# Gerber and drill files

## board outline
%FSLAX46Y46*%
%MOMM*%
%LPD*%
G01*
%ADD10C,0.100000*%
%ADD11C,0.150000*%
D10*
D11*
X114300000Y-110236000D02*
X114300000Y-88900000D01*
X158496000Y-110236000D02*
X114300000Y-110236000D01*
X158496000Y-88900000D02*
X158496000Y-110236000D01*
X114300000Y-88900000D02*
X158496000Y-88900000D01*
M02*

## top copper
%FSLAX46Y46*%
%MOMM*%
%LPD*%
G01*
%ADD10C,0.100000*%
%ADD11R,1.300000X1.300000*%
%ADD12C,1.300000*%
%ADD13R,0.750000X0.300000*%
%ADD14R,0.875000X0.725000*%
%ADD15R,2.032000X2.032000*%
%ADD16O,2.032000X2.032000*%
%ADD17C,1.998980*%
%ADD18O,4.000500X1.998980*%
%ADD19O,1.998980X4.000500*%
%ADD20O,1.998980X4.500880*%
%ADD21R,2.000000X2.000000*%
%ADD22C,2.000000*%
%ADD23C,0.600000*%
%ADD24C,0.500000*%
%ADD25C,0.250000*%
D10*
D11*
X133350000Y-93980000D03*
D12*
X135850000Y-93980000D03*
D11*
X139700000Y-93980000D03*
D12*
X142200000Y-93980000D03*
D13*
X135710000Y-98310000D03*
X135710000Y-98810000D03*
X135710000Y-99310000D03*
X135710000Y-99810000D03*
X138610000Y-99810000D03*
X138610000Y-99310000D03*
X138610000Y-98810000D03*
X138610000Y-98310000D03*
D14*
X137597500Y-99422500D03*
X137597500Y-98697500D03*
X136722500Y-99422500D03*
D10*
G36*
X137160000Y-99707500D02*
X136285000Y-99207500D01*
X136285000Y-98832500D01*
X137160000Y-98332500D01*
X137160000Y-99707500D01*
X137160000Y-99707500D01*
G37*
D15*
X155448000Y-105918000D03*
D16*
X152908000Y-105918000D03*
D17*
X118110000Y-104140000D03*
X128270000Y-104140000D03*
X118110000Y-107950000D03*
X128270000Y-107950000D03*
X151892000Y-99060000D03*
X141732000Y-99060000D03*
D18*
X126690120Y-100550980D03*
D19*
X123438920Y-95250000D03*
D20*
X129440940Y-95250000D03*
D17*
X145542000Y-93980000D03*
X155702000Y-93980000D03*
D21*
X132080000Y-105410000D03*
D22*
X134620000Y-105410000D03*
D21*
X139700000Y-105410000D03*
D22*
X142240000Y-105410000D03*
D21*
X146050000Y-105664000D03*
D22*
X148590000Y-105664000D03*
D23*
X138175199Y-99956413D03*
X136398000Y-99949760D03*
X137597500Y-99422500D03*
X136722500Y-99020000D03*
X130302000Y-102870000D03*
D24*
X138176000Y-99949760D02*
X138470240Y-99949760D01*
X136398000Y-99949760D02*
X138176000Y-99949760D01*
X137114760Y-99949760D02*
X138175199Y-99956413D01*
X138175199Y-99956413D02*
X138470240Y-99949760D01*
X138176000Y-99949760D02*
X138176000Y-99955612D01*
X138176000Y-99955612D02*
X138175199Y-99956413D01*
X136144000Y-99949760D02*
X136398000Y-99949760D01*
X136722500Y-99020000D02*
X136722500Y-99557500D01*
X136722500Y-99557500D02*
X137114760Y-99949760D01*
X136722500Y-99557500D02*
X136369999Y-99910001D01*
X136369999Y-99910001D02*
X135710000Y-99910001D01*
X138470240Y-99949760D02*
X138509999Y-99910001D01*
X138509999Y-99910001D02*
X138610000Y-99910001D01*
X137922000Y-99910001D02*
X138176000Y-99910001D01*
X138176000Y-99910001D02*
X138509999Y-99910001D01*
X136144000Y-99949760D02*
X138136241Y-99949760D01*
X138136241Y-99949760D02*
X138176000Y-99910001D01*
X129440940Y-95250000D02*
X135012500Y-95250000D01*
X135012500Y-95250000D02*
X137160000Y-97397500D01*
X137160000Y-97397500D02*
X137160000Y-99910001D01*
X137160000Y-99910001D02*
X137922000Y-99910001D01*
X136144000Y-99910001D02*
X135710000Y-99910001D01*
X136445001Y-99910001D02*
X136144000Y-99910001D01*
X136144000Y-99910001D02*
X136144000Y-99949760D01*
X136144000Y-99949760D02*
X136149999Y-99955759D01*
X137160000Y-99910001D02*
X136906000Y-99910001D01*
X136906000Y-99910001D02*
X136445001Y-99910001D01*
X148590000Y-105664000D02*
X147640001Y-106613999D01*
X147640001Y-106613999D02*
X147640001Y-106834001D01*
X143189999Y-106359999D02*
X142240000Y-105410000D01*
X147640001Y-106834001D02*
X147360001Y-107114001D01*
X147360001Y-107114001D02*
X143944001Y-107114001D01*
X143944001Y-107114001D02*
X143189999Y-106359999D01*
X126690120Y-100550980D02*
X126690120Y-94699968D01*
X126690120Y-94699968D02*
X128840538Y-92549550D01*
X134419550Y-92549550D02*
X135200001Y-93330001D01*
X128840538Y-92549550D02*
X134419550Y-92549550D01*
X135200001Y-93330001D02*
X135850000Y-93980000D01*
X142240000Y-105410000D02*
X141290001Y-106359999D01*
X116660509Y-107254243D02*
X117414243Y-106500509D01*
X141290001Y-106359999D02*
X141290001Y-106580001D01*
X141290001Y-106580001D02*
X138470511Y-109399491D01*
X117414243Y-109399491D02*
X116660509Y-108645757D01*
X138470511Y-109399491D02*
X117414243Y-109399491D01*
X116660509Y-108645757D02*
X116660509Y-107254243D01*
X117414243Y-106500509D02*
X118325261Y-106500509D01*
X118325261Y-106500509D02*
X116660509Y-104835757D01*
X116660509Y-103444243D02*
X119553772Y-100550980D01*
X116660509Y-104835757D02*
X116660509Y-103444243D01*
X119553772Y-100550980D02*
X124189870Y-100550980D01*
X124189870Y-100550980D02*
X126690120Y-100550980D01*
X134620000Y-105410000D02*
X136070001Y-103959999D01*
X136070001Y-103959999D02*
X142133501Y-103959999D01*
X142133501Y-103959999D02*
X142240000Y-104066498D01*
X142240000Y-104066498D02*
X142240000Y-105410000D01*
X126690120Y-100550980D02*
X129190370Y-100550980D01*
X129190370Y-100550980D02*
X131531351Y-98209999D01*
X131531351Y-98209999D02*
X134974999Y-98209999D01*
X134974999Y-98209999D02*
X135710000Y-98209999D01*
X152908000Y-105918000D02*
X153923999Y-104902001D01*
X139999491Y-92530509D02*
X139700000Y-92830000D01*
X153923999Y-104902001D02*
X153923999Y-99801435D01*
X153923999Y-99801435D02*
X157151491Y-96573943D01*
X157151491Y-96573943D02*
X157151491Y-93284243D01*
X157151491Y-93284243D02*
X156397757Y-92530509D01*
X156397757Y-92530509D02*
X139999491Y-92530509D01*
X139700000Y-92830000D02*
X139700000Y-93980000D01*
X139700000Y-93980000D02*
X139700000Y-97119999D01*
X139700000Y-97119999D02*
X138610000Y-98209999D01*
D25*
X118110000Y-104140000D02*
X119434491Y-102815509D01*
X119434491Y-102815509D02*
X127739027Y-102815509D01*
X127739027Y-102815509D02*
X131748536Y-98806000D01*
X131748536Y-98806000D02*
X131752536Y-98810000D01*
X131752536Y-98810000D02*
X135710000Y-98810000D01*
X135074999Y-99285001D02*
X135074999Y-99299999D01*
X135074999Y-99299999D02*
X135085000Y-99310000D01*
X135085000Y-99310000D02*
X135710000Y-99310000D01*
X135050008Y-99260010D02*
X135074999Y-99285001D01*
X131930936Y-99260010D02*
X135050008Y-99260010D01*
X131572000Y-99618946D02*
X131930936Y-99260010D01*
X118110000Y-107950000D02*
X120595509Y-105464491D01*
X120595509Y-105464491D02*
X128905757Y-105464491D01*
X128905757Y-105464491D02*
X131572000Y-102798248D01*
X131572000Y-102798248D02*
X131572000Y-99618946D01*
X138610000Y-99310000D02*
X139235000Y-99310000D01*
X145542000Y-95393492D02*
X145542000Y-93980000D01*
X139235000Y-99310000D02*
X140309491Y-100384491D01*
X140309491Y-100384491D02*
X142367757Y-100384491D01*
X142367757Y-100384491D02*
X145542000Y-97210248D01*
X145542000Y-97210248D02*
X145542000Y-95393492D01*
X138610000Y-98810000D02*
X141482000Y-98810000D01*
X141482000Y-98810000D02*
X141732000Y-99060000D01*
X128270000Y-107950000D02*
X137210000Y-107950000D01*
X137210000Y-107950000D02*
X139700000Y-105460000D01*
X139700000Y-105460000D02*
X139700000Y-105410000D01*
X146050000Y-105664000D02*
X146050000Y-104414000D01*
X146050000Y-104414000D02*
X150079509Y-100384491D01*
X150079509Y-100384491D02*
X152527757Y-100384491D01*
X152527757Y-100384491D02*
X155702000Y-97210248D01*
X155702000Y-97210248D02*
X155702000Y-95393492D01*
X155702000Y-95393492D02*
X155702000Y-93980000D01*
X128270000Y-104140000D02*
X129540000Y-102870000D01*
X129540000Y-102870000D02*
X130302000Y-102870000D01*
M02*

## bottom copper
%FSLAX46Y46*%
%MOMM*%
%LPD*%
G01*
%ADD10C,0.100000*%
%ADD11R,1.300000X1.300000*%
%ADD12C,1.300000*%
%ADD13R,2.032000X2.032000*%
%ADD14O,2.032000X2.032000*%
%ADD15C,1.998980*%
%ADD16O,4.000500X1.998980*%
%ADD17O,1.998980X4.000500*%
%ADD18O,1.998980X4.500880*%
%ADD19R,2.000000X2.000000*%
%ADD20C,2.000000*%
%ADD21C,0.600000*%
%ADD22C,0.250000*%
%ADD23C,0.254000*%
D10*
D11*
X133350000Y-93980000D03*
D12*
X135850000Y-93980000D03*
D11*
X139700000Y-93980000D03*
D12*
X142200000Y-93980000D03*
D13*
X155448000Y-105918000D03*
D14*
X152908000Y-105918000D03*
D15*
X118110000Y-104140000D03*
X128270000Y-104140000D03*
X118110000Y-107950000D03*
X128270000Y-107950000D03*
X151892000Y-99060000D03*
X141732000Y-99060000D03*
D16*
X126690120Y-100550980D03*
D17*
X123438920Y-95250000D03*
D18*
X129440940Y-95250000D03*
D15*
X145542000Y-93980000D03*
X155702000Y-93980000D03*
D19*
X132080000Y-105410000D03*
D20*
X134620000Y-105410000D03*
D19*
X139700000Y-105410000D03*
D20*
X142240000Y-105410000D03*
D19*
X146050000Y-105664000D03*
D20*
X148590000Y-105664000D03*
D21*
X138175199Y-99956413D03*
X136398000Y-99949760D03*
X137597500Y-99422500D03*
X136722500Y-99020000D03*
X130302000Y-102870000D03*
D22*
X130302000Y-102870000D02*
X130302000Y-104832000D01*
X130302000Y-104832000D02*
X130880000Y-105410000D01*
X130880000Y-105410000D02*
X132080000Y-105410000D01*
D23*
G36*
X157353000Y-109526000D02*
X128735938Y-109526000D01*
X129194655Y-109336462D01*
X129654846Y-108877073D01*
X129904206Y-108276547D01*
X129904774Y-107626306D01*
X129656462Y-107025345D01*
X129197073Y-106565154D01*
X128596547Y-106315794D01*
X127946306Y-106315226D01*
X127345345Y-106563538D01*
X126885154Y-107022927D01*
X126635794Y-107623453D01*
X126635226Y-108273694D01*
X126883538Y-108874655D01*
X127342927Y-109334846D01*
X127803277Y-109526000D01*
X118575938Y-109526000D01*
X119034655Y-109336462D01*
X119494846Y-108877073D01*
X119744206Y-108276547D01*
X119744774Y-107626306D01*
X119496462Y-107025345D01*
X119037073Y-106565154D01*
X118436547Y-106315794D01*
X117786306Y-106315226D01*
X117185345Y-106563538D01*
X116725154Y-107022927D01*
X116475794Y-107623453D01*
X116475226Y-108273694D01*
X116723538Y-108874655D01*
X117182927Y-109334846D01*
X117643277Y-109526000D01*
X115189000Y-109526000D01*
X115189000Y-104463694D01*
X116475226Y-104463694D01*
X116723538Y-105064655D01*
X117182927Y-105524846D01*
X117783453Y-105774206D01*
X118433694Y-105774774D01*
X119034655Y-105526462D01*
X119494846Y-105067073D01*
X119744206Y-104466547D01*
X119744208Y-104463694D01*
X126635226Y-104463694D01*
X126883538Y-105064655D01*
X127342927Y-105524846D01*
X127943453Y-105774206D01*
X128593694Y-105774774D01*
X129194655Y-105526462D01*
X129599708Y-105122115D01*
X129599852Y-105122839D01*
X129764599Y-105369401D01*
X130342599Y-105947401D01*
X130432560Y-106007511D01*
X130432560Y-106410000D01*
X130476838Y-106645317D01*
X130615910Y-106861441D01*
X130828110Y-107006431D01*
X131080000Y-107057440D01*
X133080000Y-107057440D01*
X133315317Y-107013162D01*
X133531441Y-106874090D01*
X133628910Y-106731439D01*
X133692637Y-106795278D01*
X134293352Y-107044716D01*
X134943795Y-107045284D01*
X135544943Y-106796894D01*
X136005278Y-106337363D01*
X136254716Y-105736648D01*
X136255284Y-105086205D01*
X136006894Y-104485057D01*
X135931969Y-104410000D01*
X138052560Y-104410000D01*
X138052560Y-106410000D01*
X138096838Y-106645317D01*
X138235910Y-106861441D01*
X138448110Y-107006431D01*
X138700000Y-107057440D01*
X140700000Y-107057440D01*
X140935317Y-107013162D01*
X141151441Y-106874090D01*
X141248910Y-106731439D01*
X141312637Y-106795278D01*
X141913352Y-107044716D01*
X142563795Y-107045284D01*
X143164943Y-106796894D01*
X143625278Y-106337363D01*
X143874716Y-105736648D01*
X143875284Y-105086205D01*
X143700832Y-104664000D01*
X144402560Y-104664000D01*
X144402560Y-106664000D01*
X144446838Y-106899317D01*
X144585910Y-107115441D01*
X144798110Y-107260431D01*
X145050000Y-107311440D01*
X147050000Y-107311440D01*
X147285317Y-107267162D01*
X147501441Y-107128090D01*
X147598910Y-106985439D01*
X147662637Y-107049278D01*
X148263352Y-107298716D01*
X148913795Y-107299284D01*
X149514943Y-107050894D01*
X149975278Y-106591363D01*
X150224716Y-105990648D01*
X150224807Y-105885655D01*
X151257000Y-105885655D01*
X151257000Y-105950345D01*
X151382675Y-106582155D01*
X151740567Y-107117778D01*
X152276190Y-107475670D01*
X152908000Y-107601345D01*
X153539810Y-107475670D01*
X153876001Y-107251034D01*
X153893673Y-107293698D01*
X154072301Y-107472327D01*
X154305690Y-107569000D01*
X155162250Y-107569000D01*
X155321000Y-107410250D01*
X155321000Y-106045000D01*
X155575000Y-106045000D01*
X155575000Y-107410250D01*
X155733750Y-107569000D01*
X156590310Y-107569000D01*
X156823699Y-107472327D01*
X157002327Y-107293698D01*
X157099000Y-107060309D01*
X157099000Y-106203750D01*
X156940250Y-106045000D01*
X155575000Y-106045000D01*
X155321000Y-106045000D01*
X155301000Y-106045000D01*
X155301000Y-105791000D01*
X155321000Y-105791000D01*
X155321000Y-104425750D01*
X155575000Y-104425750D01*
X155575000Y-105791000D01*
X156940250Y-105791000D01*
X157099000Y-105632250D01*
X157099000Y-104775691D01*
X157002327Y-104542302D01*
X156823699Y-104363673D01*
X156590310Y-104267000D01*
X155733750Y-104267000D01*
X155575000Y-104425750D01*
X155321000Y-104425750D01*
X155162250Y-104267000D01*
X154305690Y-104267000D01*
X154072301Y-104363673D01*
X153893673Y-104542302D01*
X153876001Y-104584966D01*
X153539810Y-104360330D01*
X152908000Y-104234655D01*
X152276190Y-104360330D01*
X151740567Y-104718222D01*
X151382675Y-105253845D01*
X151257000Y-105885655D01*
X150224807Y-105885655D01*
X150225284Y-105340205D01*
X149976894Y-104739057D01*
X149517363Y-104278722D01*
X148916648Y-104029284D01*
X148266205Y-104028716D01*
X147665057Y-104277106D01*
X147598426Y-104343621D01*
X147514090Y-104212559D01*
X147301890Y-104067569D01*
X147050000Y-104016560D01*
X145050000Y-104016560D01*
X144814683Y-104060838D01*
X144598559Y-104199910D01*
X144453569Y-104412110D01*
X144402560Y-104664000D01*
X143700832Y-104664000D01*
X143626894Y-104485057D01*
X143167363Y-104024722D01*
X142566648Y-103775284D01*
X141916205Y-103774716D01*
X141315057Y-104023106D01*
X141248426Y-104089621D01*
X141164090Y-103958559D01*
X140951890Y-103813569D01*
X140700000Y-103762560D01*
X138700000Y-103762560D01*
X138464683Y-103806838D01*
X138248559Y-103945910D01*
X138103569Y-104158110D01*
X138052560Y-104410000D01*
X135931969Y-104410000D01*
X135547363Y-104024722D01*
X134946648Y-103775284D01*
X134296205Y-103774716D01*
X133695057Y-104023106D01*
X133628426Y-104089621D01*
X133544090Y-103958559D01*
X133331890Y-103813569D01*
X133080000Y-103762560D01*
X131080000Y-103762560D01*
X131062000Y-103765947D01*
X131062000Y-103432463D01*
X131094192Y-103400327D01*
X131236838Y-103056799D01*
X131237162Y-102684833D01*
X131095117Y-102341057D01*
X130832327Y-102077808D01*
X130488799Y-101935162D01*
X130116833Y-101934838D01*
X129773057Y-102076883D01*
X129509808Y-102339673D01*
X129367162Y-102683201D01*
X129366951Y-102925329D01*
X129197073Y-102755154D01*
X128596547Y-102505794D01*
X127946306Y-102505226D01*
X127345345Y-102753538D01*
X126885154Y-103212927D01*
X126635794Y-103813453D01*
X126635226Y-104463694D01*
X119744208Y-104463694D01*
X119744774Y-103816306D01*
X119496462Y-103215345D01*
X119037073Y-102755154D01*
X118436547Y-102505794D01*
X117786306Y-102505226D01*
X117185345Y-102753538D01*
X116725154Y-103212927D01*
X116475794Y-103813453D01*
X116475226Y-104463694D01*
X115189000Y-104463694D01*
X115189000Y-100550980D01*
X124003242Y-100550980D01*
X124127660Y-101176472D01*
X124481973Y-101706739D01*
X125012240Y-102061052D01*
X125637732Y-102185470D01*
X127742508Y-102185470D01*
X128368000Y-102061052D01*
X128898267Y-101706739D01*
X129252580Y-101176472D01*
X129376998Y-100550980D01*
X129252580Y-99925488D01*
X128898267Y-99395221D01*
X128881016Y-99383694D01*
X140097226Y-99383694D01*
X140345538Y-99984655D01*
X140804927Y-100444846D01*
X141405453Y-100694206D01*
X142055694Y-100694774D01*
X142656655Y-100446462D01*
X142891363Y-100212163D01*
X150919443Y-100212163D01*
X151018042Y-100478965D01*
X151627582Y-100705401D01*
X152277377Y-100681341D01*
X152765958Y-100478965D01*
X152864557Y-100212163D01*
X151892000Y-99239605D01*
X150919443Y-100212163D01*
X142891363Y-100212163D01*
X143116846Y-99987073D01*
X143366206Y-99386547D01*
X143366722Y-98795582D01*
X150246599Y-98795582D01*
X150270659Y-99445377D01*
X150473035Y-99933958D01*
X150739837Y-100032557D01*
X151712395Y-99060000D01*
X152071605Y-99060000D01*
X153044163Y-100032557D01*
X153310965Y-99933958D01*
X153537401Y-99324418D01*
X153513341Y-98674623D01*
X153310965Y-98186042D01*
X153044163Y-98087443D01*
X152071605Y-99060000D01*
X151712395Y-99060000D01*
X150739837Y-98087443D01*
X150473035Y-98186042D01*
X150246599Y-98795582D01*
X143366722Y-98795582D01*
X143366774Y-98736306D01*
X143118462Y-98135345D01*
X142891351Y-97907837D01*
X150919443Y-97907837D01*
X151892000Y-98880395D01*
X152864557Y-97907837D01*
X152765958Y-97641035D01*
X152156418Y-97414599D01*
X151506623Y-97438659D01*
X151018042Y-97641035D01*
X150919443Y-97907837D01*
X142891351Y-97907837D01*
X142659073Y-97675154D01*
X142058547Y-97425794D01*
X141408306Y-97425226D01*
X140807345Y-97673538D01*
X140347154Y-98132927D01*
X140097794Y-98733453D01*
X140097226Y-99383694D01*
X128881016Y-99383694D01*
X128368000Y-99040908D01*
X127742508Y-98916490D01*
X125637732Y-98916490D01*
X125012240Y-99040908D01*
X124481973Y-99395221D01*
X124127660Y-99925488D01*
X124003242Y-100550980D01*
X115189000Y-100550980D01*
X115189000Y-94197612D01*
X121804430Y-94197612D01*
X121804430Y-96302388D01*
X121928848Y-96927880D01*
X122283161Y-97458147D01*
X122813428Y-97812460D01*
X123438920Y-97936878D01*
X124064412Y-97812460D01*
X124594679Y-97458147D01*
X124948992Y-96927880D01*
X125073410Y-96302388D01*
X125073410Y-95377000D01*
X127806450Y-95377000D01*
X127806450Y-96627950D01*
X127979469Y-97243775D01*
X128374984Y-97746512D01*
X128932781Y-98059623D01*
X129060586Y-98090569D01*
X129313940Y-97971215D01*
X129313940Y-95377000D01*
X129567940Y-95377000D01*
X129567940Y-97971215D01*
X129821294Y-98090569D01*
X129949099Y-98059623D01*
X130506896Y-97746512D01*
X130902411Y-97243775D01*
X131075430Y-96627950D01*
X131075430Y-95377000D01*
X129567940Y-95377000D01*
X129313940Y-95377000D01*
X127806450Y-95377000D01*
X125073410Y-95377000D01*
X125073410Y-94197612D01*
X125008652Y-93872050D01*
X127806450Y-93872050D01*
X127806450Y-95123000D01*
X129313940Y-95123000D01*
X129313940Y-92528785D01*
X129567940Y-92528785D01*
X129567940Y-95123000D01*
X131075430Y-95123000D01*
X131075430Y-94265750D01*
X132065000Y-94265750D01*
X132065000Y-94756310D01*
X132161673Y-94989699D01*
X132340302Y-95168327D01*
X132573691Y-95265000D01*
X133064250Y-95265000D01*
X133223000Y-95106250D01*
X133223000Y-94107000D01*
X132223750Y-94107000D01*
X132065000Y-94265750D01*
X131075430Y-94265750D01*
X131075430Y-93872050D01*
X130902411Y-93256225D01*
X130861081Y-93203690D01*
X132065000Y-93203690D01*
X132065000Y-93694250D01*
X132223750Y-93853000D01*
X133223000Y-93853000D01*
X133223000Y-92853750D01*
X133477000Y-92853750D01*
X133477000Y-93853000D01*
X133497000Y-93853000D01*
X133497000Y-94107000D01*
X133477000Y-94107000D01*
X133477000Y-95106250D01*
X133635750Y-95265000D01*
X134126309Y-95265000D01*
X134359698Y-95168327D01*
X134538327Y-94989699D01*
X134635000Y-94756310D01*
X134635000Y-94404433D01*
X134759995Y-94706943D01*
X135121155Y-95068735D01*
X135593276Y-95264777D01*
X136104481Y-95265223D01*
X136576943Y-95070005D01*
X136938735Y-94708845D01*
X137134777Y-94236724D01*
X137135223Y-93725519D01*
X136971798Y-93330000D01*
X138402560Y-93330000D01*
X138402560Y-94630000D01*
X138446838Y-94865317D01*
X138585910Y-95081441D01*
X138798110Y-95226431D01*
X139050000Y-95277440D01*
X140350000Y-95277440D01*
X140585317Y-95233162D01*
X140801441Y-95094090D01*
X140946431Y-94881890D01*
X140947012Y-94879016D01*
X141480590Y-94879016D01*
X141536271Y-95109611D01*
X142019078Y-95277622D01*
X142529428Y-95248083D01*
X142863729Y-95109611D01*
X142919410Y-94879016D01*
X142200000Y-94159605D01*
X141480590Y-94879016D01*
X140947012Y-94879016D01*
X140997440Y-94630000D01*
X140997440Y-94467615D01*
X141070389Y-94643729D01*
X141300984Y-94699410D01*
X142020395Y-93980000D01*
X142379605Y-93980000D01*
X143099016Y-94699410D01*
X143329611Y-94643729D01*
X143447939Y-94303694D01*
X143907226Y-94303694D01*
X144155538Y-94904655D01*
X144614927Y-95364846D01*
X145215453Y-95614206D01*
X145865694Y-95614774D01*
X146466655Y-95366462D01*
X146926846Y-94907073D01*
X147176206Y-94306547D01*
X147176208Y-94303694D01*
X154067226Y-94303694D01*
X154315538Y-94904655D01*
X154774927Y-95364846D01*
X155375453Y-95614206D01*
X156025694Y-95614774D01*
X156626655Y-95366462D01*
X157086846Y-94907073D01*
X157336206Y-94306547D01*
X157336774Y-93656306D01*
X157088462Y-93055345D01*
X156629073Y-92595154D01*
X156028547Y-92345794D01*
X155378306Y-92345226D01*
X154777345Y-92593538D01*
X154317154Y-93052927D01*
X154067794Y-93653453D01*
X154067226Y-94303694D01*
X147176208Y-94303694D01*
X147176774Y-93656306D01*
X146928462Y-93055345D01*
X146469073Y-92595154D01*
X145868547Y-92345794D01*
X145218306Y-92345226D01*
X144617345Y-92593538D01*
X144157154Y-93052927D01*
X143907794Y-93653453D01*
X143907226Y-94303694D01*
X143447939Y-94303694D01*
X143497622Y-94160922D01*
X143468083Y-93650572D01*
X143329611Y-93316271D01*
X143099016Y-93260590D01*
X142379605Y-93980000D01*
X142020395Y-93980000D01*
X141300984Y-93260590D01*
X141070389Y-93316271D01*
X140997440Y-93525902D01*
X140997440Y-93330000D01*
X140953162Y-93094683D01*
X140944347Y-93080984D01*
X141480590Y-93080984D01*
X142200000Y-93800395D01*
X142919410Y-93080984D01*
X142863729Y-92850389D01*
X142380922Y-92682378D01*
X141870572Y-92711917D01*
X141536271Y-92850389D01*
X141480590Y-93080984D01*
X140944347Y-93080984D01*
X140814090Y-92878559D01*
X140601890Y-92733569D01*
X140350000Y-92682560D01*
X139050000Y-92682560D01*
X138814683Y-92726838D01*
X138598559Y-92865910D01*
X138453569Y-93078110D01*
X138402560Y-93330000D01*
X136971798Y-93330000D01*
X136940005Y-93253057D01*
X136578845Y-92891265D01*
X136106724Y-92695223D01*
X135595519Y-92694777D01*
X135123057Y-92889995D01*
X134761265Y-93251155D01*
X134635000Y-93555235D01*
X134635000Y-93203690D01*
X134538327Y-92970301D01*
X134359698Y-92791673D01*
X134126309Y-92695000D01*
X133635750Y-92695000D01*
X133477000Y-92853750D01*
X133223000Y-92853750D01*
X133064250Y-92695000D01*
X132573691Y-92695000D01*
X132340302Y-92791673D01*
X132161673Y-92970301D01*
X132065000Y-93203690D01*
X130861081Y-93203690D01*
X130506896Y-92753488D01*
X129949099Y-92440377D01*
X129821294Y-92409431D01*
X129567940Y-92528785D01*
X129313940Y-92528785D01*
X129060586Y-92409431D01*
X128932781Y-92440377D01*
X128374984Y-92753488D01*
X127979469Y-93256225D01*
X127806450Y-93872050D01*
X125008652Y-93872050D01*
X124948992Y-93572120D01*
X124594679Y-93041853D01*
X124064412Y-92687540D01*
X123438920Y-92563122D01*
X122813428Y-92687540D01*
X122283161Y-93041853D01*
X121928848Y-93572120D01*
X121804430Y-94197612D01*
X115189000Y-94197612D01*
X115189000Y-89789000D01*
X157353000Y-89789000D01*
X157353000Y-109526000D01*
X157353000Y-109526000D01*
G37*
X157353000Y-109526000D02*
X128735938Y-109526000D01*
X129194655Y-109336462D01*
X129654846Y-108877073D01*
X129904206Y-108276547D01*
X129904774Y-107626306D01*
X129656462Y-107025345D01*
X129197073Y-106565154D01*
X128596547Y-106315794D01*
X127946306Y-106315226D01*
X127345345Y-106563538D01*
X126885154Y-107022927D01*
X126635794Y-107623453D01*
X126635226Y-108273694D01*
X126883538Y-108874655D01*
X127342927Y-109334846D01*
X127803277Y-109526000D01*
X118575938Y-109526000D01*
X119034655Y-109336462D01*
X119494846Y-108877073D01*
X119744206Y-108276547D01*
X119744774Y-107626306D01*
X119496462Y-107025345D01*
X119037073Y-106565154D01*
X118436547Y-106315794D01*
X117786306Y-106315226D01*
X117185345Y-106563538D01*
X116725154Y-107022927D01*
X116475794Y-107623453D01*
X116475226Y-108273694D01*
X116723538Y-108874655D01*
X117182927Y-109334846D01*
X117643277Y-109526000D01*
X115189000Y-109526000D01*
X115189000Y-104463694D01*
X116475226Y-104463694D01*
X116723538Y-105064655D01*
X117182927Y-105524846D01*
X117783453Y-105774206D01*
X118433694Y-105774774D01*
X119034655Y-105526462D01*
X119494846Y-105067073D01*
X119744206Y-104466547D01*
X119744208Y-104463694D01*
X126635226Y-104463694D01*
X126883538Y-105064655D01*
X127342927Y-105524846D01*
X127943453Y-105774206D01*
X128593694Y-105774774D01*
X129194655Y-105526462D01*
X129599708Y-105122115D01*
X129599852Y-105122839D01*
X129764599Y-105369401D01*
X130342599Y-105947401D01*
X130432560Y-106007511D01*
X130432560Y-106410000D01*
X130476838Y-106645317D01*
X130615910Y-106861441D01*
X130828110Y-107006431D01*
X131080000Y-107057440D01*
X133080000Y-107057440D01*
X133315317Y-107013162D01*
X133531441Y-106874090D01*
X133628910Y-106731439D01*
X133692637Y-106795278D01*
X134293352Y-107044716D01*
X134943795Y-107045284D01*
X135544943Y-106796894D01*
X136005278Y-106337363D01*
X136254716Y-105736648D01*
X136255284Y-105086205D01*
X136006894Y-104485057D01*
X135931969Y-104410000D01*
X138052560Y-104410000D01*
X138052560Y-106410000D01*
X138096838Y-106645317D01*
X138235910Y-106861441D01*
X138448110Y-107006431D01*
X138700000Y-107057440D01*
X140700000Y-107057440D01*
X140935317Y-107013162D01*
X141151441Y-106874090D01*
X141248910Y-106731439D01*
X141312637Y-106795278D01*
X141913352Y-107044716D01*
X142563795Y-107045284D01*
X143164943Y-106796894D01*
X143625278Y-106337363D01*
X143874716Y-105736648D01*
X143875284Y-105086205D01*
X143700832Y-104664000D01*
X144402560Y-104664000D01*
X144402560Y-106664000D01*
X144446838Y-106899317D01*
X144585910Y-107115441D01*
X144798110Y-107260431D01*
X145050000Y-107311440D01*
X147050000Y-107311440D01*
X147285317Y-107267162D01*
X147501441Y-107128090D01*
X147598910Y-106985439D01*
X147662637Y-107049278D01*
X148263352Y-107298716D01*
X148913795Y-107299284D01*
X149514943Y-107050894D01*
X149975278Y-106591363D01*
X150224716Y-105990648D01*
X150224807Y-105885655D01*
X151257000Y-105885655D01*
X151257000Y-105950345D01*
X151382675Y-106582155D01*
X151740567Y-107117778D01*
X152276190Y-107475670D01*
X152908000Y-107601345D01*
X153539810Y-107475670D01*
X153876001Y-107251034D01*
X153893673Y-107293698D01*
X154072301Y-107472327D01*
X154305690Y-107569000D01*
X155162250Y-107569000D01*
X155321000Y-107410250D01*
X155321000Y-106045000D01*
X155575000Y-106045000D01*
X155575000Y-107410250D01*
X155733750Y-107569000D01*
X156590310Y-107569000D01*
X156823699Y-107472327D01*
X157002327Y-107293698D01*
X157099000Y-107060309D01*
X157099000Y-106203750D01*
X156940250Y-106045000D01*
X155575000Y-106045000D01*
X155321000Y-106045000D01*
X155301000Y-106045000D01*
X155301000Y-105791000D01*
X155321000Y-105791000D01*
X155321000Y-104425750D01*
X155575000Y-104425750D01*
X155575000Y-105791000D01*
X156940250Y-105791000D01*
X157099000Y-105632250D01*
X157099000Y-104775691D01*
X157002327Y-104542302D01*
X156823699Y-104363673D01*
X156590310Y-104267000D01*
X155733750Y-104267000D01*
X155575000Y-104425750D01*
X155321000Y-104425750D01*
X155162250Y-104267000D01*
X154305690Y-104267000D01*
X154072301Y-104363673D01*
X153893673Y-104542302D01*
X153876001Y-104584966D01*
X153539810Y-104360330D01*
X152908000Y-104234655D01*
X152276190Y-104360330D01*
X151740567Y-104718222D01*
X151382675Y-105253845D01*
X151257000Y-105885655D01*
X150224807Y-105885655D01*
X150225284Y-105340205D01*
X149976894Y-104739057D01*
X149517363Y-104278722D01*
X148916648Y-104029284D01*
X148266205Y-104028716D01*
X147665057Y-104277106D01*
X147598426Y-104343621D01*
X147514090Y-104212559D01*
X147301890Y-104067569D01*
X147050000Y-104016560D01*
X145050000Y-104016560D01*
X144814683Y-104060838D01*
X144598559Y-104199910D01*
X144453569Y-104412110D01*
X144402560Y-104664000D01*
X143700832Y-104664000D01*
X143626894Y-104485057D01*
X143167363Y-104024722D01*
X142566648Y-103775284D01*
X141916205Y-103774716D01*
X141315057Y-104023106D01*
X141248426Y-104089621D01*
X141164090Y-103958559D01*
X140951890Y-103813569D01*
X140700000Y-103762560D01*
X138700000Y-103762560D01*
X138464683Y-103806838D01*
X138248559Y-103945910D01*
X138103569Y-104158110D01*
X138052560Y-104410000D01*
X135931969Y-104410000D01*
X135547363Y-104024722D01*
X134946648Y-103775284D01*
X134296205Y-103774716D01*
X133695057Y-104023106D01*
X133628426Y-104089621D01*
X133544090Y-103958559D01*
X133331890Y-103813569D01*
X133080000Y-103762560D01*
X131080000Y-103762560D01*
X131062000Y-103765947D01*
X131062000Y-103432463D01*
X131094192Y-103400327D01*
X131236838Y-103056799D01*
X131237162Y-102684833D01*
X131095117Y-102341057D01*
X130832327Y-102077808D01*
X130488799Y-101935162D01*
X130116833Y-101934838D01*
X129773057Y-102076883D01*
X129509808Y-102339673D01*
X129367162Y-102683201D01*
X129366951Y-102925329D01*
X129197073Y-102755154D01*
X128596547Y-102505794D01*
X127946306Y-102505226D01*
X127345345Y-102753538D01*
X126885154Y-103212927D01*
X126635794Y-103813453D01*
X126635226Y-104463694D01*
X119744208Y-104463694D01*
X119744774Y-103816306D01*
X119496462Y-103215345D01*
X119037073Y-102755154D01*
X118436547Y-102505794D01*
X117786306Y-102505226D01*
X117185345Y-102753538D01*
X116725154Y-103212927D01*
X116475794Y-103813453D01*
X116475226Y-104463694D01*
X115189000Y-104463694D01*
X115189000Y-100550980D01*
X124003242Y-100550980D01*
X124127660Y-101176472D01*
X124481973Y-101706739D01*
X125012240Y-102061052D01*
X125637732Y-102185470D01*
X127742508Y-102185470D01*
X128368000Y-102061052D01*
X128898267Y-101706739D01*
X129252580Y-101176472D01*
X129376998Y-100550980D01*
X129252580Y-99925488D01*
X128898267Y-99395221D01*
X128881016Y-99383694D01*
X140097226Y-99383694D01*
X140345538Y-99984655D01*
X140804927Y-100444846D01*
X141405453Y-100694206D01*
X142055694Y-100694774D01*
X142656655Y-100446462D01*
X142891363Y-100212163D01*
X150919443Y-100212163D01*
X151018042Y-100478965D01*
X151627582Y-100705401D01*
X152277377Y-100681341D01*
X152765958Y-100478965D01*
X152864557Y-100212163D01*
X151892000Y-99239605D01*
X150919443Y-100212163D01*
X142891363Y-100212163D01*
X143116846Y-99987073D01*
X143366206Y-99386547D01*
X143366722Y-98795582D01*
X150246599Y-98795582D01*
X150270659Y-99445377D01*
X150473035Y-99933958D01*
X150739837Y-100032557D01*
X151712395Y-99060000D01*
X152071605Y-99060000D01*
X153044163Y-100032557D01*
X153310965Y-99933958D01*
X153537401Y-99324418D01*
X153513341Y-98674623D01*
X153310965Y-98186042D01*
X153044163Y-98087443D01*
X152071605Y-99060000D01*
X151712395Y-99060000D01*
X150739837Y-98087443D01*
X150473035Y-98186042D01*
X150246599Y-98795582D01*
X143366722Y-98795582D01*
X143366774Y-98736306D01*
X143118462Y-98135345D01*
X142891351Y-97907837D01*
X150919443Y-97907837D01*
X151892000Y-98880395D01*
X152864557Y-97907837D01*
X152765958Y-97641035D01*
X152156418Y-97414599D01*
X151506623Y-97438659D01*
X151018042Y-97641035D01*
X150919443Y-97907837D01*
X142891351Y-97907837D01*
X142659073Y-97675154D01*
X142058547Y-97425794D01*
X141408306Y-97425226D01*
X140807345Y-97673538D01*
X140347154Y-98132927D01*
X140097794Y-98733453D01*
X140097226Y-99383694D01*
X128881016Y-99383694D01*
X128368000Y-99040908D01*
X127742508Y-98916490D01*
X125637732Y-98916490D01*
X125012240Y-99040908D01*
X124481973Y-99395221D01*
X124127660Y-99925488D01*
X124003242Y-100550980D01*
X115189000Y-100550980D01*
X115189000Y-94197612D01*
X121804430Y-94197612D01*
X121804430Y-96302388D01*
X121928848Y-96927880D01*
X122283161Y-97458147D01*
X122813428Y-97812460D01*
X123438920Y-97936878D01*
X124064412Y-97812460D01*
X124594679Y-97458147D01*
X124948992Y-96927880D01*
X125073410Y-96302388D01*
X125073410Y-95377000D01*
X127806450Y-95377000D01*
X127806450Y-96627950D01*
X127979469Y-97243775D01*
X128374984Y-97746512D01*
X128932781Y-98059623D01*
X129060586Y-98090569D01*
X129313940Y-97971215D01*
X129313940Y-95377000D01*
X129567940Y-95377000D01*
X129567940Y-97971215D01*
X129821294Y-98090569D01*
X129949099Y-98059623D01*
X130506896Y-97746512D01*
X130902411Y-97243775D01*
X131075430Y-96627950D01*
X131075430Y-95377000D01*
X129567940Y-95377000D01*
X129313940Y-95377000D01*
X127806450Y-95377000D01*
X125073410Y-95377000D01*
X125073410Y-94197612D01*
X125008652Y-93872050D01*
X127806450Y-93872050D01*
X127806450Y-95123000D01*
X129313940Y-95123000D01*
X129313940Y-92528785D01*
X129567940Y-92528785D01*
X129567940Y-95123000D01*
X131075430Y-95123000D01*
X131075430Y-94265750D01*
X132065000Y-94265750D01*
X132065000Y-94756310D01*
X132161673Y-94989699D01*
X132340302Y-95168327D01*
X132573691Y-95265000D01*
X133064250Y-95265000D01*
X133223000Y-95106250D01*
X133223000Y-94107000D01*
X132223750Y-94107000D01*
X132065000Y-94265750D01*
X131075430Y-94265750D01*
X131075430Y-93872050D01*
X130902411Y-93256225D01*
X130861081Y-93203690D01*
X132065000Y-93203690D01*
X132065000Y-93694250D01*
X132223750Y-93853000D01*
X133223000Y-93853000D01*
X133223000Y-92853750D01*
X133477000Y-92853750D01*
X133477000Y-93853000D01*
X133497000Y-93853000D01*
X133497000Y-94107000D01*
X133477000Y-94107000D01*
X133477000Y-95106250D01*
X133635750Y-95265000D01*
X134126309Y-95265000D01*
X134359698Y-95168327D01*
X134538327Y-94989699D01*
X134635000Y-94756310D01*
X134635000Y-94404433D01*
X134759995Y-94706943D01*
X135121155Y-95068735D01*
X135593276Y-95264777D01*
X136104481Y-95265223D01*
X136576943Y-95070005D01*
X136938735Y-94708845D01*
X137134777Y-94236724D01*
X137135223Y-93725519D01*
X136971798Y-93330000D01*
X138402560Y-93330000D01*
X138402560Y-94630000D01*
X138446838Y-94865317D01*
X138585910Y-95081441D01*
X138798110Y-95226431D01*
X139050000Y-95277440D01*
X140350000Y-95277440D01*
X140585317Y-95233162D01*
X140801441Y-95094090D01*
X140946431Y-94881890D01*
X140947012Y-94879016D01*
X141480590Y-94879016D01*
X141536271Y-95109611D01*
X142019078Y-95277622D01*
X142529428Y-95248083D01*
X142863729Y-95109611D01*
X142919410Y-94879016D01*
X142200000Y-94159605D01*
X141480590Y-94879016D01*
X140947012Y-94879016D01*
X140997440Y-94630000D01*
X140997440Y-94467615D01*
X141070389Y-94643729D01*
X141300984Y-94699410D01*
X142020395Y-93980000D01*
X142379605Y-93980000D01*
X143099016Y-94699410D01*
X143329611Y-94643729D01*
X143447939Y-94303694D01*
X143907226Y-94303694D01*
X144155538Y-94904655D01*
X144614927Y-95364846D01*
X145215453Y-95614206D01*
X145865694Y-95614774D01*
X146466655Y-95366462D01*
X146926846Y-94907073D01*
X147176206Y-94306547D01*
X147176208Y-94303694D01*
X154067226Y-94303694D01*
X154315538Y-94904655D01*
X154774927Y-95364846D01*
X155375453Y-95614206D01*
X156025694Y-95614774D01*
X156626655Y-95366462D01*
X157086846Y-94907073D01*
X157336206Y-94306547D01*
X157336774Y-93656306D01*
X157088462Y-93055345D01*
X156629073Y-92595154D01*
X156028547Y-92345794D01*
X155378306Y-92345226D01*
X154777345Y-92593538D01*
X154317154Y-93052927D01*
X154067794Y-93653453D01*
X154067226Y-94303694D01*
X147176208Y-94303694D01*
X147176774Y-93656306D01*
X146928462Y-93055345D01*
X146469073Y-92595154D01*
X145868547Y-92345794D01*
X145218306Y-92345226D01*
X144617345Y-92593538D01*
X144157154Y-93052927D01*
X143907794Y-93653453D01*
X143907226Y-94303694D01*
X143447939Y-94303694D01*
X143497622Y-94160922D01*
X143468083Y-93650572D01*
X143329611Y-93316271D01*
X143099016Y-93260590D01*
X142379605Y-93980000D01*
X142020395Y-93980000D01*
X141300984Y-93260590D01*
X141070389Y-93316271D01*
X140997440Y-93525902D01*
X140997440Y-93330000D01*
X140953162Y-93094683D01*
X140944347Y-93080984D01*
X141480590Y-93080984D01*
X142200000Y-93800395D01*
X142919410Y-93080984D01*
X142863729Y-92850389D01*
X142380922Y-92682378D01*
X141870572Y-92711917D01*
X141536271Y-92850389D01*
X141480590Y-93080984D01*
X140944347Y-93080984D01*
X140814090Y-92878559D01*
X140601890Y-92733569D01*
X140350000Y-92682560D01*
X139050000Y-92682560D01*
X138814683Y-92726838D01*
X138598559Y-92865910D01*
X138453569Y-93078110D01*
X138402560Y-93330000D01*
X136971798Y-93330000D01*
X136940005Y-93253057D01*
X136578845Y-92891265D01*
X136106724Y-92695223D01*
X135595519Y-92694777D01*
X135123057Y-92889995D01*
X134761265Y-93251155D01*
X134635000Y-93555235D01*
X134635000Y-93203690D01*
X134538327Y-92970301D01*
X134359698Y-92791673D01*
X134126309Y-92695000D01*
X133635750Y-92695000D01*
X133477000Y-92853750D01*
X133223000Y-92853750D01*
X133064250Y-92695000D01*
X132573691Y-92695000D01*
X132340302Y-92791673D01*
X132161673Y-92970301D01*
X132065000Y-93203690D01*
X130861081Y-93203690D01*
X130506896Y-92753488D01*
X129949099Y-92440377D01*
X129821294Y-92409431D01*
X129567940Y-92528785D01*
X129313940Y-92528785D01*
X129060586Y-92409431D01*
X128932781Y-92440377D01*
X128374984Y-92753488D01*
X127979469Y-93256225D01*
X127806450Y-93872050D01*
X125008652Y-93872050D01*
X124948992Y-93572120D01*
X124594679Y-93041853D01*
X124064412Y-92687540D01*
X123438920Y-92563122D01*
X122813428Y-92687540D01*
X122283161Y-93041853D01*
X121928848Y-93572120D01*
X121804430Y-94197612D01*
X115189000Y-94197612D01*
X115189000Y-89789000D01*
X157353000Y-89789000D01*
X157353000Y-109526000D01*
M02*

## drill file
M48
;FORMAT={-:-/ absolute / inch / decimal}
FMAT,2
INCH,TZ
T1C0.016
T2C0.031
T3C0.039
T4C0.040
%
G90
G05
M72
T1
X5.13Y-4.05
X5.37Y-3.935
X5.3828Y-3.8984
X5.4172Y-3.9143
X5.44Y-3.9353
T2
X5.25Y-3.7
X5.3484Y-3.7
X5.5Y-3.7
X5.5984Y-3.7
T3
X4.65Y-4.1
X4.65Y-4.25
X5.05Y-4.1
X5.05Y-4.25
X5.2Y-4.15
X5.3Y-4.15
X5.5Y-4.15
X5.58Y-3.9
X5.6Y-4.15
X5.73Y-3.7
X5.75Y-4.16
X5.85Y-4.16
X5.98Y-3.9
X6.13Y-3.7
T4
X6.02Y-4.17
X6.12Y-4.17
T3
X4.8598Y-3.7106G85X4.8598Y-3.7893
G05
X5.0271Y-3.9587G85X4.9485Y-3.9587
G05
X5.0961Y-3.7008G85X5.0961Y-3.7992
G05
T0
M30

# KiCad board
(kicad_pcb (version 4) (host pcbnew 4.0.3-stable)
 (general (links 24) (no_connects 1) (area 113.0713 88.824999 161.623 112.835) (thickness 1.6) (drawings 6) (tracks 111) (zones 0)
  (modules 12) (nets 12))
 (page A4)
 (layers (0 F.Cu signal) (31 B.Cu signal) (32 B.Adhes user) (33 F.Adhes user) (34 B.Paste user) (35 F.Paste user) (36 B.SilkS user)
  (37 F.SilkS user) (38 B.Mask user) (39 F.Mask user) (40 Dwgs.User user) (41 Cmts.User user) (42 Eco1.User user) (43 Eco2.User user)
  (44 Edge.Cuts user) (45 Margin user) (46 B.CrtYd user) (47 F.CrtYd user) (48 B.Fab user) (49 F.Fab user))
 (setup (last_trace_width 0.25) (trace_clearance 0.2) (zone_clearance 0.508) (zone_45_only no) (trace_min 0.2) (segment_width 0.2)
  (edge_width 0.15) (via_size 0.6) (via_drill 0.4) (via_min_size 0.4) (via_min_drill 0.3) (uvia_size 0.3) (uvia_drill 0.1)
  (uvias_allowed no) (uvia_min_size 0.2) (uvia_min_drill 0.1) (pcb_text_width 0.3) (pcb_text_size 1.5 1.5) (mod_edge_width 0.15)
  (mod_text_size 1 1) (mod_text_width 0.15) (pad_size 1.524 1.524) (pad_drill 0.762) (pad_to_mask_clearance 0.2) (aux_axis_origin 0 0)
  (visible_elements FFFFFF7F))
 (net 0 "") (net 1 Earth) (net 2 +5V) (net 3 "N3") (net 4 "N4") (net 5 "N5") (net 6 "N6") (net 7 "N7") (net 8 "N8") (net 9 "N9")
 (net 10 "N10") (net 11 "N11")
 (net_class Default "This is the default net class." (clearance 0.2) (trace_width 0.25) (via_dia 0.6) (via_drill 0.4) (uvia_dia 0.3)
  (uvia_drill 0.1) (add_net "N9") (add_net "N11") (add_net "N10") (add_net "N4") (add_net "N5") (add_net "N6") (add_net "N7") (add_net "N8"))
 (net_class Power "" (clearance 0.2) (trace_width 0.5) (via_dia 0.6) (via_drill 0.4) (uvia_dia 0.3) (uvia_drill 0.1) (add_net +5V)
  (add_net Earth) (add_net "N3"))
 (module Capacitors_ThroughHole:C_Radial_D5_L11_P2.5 (layer F.Cu) (at 133.35 93.98)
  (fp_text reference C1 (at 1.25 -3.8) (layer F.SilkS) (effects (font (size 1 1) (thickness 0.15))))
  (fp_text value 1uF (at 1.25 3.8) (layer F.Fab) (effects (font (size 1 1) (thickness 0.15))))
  (pad 1 thru_hole rect (at 0 0) (size 1.3 1.3) (drill 0.8) (layers *.Cu *.Mask F.SilkS) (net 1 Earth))
  (pad 2 thru_hole circle (at 2.5 0) (size 1.3 1.3) (drill 0.8) (layers *.Cu *.Mask F.SilkS) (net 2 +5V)))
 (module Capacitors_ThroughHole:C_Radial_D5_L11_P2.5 (layer F.Cu) (at 139.7 93.98)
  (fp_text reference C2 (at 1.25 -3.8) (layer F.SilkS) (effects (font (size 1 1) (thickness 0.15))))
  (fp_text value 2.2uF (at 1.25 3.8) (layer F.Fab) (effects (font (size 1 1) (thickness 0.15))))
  (pad 1 thru_hole rect (at 0 0) (size 1.3 1.3) (drill 0.8) (layers *.Cu *.Mask F.SilkS) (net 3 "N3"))
  (pad 2 thru_hole circle (at 2.5 0) (size 1.3 1.3) (drill 0.8) (layers *.Cu *.Mask F.SilkS) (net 1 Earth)))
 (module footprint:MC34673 (layer F.Cu) (at 137.16 99.06)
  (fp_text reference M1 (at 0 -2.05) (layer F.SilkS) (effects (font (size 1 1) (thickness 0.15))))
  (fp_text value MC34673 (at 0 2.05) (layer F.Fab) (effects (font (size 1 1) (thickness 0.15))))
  (pad 1 smd rect (at -1.45 -0.75) (size 0.75 0.3) (layers F.Cu F.Paste F.Mask) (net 2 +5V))
  (pad 2 smd rect (at -1.45 -0.25) (size 0.75 0.3) (layers F.Cu F.Paste F.Mask) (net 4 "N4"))
  (pad 3 smd rect (at -1.45 0.25) (size 0.75 0.3) (layers F.Cu F.Paste F.Mask) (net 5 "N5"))
  (pad 4 smd rect (at -1.45 0.75) (size 0.75 0.3) (layers F.Cu F.Paste F.Mask) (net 1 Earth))
  (pad 5 smd rect (at 1.45 0.75) (size 0.75 0.3) (layers F.Cu F.Paste F.Mask) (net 1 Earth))
  (pad 6 smd rect (at 1.45 0.25) (size 0.75 0.3) (layers F.Cu F.Paste F.Mask) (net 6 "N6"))
  (pad 7 smd rect (at 1.45 -0.25) (size 0.75 0.3) (layers F.Cu F.Paste F.Mask) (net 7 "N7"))
  (pad 8 smd rect (at 1.45 -0.75) (size 0.75 0.3) (layers F.Cu F.Paste F.Mask) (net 3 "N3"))
  (pad 5 smd rect (at 0.4375 0.3625) (size 0.875 0.725) (layers F.Cu F.Paste F.Mask) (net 1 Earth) (solder_paste_margin_ratio -0.2))
  (pad 5 smd rect (at 0.4375 -0.3625) (size 0.875 0.725) (layers F.Cu F.Paste F.Mask) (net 1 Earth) (solder_paste_margin_ratio -0.2))
  (pad 5 smd rect (at -0.4375 0.3625) (size 0.875 0.725) (layers F.Cu F.Paste F.Mask) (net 1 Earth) (solder_paste_margin_ratio -0.2))
  (pad 5 smd trapezoid (at -0.4375 -0.04 90) (size 0.875 0.875) (rect_delta 0 0.5) (layers F.Cu F.Paste F.Mask) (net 1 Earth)
   (solder_paste_margin_ratio -0.2)))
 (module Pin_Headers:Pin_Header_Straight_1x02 (layer F.Cu) (at 155.448 105.918 270)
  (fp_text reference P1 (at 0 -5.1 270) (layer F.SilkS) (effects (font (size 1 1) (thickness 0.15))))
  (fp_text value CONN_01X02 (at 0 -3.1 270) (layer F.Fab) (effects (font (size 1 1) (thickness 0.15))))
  (pad 1 thru_hole rect (at 0 0 270) (size 2.032 2.032) (drill 1.016) (layers *.Cu *.Mask F.SilkS) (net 1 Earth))
  (pad 2 thru_hole oval (at 0 2.54 270) (size 2.032 2.032) (drill 1.016) (layers *.Cu *.Mask F.SilkS) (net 3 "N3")))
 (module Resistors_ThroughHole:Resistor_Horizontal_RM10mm (layer F.Cu) (at 118.11 104.14)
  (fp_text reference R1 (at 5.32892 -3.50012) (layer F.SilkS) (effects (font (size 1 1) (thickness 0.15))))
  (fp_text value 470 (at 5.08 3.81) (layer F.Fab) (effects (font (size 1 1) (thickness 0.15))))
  (pad 1 thru_hole circle (at 0 0) (size 1.99898 1.99898) (drill 1.00076) (layers *.Cu *.SilkS *.Mask) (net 4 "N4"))
  (pad 2 thru_hole circle (at 10.16 0) (size 1.99898 1.99898) (drill 1.00076) (layers *.Cu *.SilkS *.Mask) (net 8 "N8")))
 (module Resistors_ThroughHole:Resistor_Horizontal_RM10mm (layer F.Cu) (at 118.11 107.95)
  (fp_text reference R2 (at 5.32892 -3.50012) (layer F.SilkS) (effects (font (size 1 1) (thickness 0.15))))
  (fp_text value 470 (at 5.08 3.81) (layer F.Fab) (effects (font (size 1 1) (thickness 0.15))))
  (pad 1 thru_hole circle (at 0 0) (size 1.99898 1.99898) (drill 1.00076) (layers *.Cu *.SilkS *.Mask) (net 5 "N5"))
  (pad 2 thru_hole circle (at 10.16 0) (size 1.99898 1.99898) (drill 1.00076) (layers *.Cu *.SilkS *.Mask) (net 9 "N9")))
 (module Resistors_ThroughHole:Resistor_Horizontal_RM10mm (layer F.Cu) (at 151.892 99.06 180)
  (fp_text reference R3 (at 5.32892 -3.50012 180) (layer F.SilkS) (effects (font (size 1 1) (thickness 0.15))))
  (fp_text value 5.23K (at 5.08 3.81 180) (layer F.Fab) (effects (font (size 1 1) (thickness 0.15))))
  (pad 1 thru_hole circle (at 0 0 180) (size 1.99898 1.99898) (drill 1.00076) (layers *.Cu *.SilkS *.Mask) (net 1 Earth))
  (pad 2 thru_hole circle (at 10.16 0 180) (size 1.99898 1.99898) (drill 1.00076) (layers *.Cu *.SilkS *.Mask) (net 7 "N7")))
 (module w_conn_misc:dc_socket (layer F.Cu) (at 123.19 95.25 270)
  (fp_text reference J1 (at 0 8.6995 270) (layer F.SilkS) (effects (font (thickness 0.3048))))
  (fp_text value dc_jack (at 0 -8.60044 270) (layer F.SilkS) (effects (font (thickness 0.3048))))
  (pad 1 thru_hole oval (at 5.30098 -3.50012 270) (size 1.99898 4.0005) (drill oval 1.00076 2.99974) (layers *.Cu *.Mask F.SilkS)
   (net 2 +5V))
  (pad 2 thru_hole oval (at 0 -0.24892 270) (size 4.0005 1.99898) (drill oval 2.99974 1.00076) (layers *.Cu *.Mask F.SilkS) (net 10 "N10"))
  (pad 3 thru_hole oval (at 0 -6.25094 270) (size 4.50088 1.99898) (drill oval 3.50012 1.00076) (layers *.Cu *.Mask F.SilkS) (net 1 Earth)))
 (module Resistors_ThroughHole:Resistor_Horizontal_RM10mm (layer F.Cu) (at 145.542 93.98)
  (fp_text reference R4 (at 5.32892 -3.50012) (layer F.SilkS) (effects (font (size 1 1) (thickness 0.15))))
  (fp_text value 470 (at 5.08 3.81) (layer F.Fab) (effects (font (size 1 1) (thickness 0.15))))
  (pad 1 thru_hole circle (at 0 0) (size 1.99898 1.99898) (drill 1.00076) (layers *.Cu *.SilkS *.Mask) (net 6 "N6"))
  (pad 2 thru_hole circle (at 10.16 0) (size 1.99898 1.99898) (drill 1.00076) (layers *.Cu *.SilkS *.Mask) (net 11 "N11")))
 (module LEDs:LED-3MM (layer F.Cu) (at 132.08 105.41)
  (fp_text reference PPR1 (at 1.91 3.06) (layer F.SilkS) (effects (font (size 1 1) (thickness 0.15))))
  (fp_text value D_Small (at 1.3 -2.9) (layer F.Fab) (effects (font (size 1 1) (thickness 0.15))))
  (pad 1 thru_hole rect (at 0 0 90) (size 2 2) (drill 1.00076) (layers *.Cu *.Mask F.SilkS) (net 8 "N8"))
  (pad 2 thru_hole circle (at 2.54 0) (size 2 2) (drill 1.00076) (layers *.Cu *.Mask F.SilkS) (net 2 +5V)))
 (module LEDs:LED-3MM (layer F.Cu) (at 139.7 105.41)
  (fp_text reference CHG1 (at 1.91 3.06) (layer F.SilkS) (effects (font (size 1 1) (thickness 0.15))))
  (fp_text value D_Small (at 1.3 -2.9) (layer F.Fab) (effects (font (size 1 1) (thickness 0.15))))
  (pad 1 thru_hole rect (at 0 0 90) (size 2 2) (drill 1.00076) (layers *.Cu *.Mask F.SilkS) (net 9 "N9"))
  (pad 2 thru_hole circle (at 2.54 0) (size 2 2) (drill 1.00076) (layers *.Cu *.Mask F.SilkS) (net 2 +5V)))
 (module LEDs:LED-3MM (layer F.Cu) (at 146.05 105.664)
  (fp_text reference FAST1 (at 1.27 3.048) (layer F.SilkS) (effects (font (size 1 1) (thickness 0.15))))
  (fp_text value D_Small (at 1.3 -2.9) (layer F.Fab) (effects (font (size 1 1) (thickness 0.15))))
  (pad 1 thru_hole rect (at 0 0 90) (size 2 2) (drill 1.00076) (layers *.Cu *.Mask F.SilkS) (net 11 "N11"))
  (pad 2 thru_hole circle (at 2.54 0) (size 2 2) (drill 1.00076) (layers *.Cu *.Mask F.SilkS) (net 2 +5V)))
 (gr_line (start 114.3 110.236) (end 114.3 88.9) (layer Edge.Cuts) (width 0.15))
 (gr_line (start 158.496 110.236) (end 114.3 110.236) (layer Edge.Cuts) (width 0.15))
 (gr_line (start 158.496 88.9) (end 158.496 110.236) (layer Edge.Cuts) (width 0.15))
 (gr_line (start 114.3 88.9) (end 158.496 88.9) (layer Edge.Cuts) (width 0.15))
 (segment (start 138.176 99.94976) (end 138.47024 99.94976) (width 0.5) (layer F.Cu) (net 1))
 (segment (start 136.398 99.94976) (end 138.176 99.94976) (width 0.5) (layer F.Cu) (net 1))
 (segment (start 137.11476 99.94976) (end 138.175199 99.956413) (width 0.5) (layer F.Cu) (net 1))
 (segment (start 138.175199 99.956413) (end 138.47024 99.94976) (width 0.5) (layer F.Cu) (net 1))
 (segment (start 138.176 99.94976) (end 138.176 99.955612) (width 0.5) (layer F.Cu) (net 1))
 (segment (start 138.176 99.955612) (end 138.175199 99.956413) (width 0.5) (layer F.Cu) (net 1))
 (via (at 138.175199 99.956413) (size 0.6) (drill 0.4) (layers F.Cu B.Cu) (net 1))
 (segment (start 136.144 99.94976) (end 136.398 99.94976) (width 0.5) (layer F.Cu) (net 1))
 (via (at 136.398 99.94976) (size 0.6) (drill 0.4) (layers F.Cu B.Cu) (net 1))
 (via (at 137.5975 99.4225) (size 0.6) (drill 0.4) (layers F.Cu B.Cu) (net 1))
 (via (at 136.7225 99.02) (size 0.6) (drill 0.4) (layers F.Cu B.Cu) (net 1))
 (segment (start 136.7225 99.02) (end 136.7225 99.5575) (width 0.5) (layer F.Cu) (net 1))
 (segment (start 136.7225 99.5575) (end 137.11476 99.94976) (width 0.5) (layer F.Cu) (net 1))
 (segment (start 136.7225 99.5575) (end 136.369999 99.910001) (width 0.5) (layer F.Cu) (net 1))
 (segment (start 136.369999 99.910001) (end 135.71 99.910001) (width 0.5) (layer F.Cu) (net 1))
 (segment (start 138.47024 99.94976) (end 138.509999 99.910001) (width 0.5) (layer F.Cu) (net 1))
 (segment (start 138.509999 99.910001) (end 138.61 99.910001) (width 0.5) (layer F.Cu) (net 1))
 (segment (start 137.922 99.910001) (end 138.176 99.910001) (width 0.5) (layer F.Cu) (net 1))
 (segment (start 138.176 99.910001) (end 138.509999 99.910001) (width 0.5) (layer F.Cu) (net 1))
 (segment (start 136.144 99.94976) (end 138.136241 99.94976) (width 0.5) (layer F.Cu) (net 1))
 (segment (start 138.136241 99.94976) (end 138.176 99.910001) (width 0.5) (layer F.Cu) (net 1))
 (segment (start 129.44094 95.25) (end 135.0125 95.25) (width 0.5) (layer F.Cu) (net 1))
 (segment (start 135.0125 95.25) (end 137.16 97.3975) (width 0.5) (layer F.Cu) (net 1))
 (segment (start 137.16 97.3975) (end 137.16 99.910001) (width 0.5) (layer F.Cu) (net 1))
 (segment (start 137.16 99.910001) (end 137.922 99.910001) (width 0.5) (layer F.Cu) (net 1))
 (segment (start 136.144 99.910001) (end 135.71 99.910001) (width 0.5) (layer F.Cu) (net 1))
 (segment (start 136.445001 99.910001) (end 136.144 99.910001) (width 0.5) (layer F.Cu) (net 1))
 (segment (start 136.144 99.910001) (end 136.144 99.94976) (width 0.5) (layer F.Cu) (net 1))
 (segment (start 136.144 99.94976) (end 136.149999 99.955759) (width 0.5) (layer F.Cu) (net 1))
 (segment (start 137.16 99.910001) (end 136.906 99.910001) (width 0.5) (layer F.Cu) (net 1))
 (segment (start 136.906 99.910001) (end 136.445001 99.910001) (width 0.5) (layer F.Cu) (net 1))
 (segment (start 148.59 105.664) (end 147.640001 106.613999) (width 0.5) (layer F.Cu) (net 2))
 (segment (start 147.640001 106.613999) (end 147.640001 106.834001) (width 0.5) (layer F.Cu) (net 2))
 (segment (start 143.189999 106.359999) (end 142.24 105.41) (width 0.5) (layer F.Cu) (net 2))
 (segment (start 147.640001 106.834001) (end 147.360001 107.114001) (width 0.5) (layer F.Cu) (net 2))
 (segment (start 147.360001 107.114001) (end 143.944001 107.114001) (width 0.5) (layer F.Cu) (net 2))
 (segment (start 143.944001 107.114001) (end 143.189999 106.359999) (width 0.5) (layer F.Cu) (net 2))
 (segment (start 126.69012 100.55098) (end 126.69012 94.699968) (width 0.5) (layer F.Cu) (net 2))
 (segment (start 126.69012 94.699968) (end 128.840538 92.54955) (width 0.5) (layer F.Cu) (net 2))
 (segment (start 134.41955 92.54955) (end 135.200001 93.330001) (width 0.5) (layer F.Cu) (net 2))
 (segment (start 128.840538 92.54955) (end 134.41955 92.54955) (width 0.5) (layer F.Cu) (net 2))
 (segment (start 135.200001 93.330001) (end 135.85 93.98) (width 0.5) (layer F.Cu) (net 2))
 (segment (start 142.24 105.41) (end 141.290001 106.359999) (width 0.5) (layer F.Cu) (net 2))
 (segment (start 116.660509 107.254243) (end 117.414243 106.500509) (width 0.5) (layer F.Cu) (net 2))
 (segment (start 141.290001 106.359999) (end 141.290001 106.580001) (width 0.5) (layer F.Cu) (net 2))
 (segment (start 141.290001 106.580001) (end 138.470511 109.399491) (width 0.5) (layer F.Cu) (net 2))
 (segment (start 117.414243 109.399491) (end 116.660509 108.645757) (width 0.5) (layer F.Cu) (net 2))
 (segment (start 138.470511 109.399491) (end 117.414243 109.399491) (width 0.5) (layer F.Cu) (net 2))
 (segment (start 116.660509 108.645757) (end 116.660509 107.254243) (width 0.5) (layer F.Cu) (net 2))
 (segment (start 117.414243 106.500509) (end 118.325261 106.500509) (width 0.5) (layer F.Cu) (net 2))
 (segment (start 118.325261 106.500509) (end 116.660509 104.835757) (width 0.5) (layer F.Cu) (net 2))
 (segment (start 116.660509 103.444243) (end 119.553772 100.55098) (width 0.5) (layer F.Cu) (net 2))
 (segment (start 116.660509 104.835757) (end 116.660509 103.444243) (width 0.5) (layer F.Cu) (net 2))
 (segment (start 119.553772 100.55098) (end 124.18987 100.55098) (width 0.5) (layer F.Cu) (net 2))
 (segment (start 124.18987 100.55098) (end 126.69012 100.55098) (width 0.5) (layer F.Cu) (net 2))
 (segment (start 134.62 105.41) (end 136.070001 103.959999) (width 0.5) (layer F.Cu) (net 2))
 (segment (start 136.070001 103.959999) (end 142.133501 103.959999) (width 0.5) (layer F.Cu) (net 2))
 (segment (start 142.133501 103.959999) (end 142.24 104.066498) (width 0.5) (layer F.Cu) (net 2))
 (segment (start 142.24 104.066498) (end 142.24 105.41) (width 0.5) (layer F.Cu) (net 2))
 (segment (start 126.69012 100.55098) (end 129.19037 100.55098) (width 0.5) (layer F.Cu) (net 2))
 (segment (start 129.19037 100.55098) (end 131.531351 98.209999) (width 0.5) (layer F.Cu) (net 2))
 (segment (start 131.531351 98.209999) (end 134.974999 98.209999) (width 0.5) (layer F.Cu) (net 2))
 (segment (start 134.974999 98.209999) (end 135.71 98.209999) (width 0.5) (layer F.Cu) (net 2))
 (segment (start 152.908 105.918) (end 153.923999 104.902001) (width 0.5) (layer F.Cu) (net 3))
 (segment (start 139.999491 92.530509) (end 139.7 92.83) (width 0.5) (layer F.Cu) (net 3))
 (segment (start 153.923999 104.902001) (end 153.923999 99.801435) (width 0.5) (layer F.Cu) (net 3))
 (segment (start 153.923999 99.801435) (end 157.151491 96.573943) (width 0.5) (layer F.Cu) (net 3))
 (segment (start 157.151491 96.573943) (end 157.151491 93.284243) (width 0.5) (layer F.Cu) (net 3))
 (segment (start 157.151491 93.284243) (end 156.397757 92.530509) (width 0.5) (layer F.Cu) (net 3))
 (segment (start 156.397757 92.530509) (end 139.999491 92.530509) (width 0.5) (layer F.Cu) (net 3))
 (segment (start 139.7 92.83) (end 139.7 93.98) (width 0.5) (layer F.Cu) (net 3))
 (segment (start 139.7 93.98) (end 139.7 97.119999) (width 0.5) (layer F.Cu) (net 3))
 (segment (start 139.7 97.119999) (end 138.61 98.209999) (width 0.5) (layer F.Cu) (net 3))
 (segment (start 118.11 104.14) (end 119.434491 102.815509) (width 0.25) (layer F.Cu) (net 4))
 (segment (start 119.434491 102.815509) (end 127.739027 102.815509) (width 0.25) (layer F.Cu) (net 4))
 (segment (start 127.739027 102.815509) (end 131.748536 98.806) (width 0.25) (layer F.Cu) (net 4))
 (segment (start 131.748536 98.806) (end 131.752536 98.81) (width 0.25) (layer F.Cu) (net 4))
 (segment (start 131.752536 98.81) (end 135.71 98.81) (width 0.25) (layer F.Cu) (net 4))
 (segment (start 135.074999 99.285001) (end 135.074999 99.299999) (width 0.25) (layer F.Cu) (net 5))
 (segment (start 135.074999 99.299999) (end 135.085 99.31) (width 0.25) (layer F.Cu) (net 5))
 (segment (start 135.085 99.31) (end 135.71 99.31) (width 0.25) (layer F.Cu) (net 5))
 (segment (start 135.050008 99.26001) (end 135.074999 99.285001) (width 0.25) (layer F.Cu) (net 5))
 (segment (start 131.930936 99.26001) (end 135.050008 99.26001) (width 0.25) (layer F.Cu) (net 5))
 (segment (start 131.572 99.618946) (end 131.930936 99.26001) (width 0.25) (layer F.Cu) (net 5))
 (segment (start 118.11 107.95) (end 120.595509 105.464491) (width 0.25) (layer F.Cu) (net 5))
 (segment (start 120.595509 105.464491) (end 128.905757 105.464491) (width 0.25) (layer F.Cu) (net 5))
 (segment (start 128.905757 105.464491) (end 131.572 102.798248) (width 0.25) (layer F.Cu) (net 5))
 (segment (start 131.572 102.798248) (end 131.572 99.618946) (width 0.25) (layer F.Cu) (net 5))
 (segment (start 138.61 99.31) (end 139.235 99.31) (width 0.25) (layer F.Cu) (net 6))
 (segment (start 145.542 95.393492) (end 145.542 93.98) (width 0.25) (layer F.Cu) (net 6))
 (segment (start 139.235 99.31) (end 140.309491 100.384491) (width 0.25) (layer F.Cu) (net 6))
 (segment (start 140.309491 100.384491) (end 142.367757 100.384491) (width 0.25) (layer F.Cu) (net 6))
 (segment (start 142.367757 100.384491) (end 145.542 97.210248) (width 0.25) (layer F.Cu) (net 6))
 (segment (start 145.542 97.210248) (end 145.542 95.393492) (width 0.25) (layer F.Cu) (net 6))
 (segment (start 138.61 98.81) (end 141.482 98.81) (width 0.25) (layer F.Cu) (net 7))
 (segment (start 141.482 98.81) (end 141.732 99.06) (width 0.25) (layer F.Cu) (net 7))
 (segment (start 128.27 107.95) (end 137.21 107.95) (width 0.25) (layer F.Cu) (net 9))
 (segment (start 137.21 107.95) (end 139.7 105.46) (width 0.25) (layer F.Cu) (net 9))
 (segment (start 139.7 105.46) (end 139.7 105.41) (width 0.25) (layer F.Cu) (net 9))
 (segment (start 146.05 105.664) (end 146.05 104.414) (width 0.25) (layer F.Cu) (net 11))
 (segment (start 146.05 104.414) (end 150.079509 100.384491) (width 0.25) (layer F.Cu) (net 11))
 (segment (start 150.079509 100.384491) (end 152.527757 100.384491) (width 0.25) (layer F.Cu) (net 11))
 (segment (start 152.527757 100.384491) (end 155.702 97.210248) (width 0.25) (layer F.Cu) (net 11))
 (segment (start 155.702 97.210248) (end 155.702 95.393492) (width 0.25) (layer F.Cu) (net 11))
 (segment (start 155.702 95.393492) (end 155.702 93.98) (width 0.25) (layer F.Cu) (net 11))
 (segment (start 130.302 102.87) (end 130.302 104.832) (width 0.25) (layer B.Cu) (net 8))
 (segment (start 130.302 104.832) (end 130.88 105.41) (width 0.25) (layer B.Cu) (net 8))
 (segment (start 130.88 105.41) (end 132.08 105.41) (width 0.25) (layer B.Cu) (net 8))
 (segment (start 128.27 104.14) (end 129.54 102.87) (width 0.25) (layer F.Cu) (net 8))
 (segment (start 129.54 102.87) (end 130.302 102.87) (width 0.25) (layer F.Cu) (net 8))
 (via (at 130.302 102.87) (size 0.6) (drill 0.4) (layers F.Cu B.Cu) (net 8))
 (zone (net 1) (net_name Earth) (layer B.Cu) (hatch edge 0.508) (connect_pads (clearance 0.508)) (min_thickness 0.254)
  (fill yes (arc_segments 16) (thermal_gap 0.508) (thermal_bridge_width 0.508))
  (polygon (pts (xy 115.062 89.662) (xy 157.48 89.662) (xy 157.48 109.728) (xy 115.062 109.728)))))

